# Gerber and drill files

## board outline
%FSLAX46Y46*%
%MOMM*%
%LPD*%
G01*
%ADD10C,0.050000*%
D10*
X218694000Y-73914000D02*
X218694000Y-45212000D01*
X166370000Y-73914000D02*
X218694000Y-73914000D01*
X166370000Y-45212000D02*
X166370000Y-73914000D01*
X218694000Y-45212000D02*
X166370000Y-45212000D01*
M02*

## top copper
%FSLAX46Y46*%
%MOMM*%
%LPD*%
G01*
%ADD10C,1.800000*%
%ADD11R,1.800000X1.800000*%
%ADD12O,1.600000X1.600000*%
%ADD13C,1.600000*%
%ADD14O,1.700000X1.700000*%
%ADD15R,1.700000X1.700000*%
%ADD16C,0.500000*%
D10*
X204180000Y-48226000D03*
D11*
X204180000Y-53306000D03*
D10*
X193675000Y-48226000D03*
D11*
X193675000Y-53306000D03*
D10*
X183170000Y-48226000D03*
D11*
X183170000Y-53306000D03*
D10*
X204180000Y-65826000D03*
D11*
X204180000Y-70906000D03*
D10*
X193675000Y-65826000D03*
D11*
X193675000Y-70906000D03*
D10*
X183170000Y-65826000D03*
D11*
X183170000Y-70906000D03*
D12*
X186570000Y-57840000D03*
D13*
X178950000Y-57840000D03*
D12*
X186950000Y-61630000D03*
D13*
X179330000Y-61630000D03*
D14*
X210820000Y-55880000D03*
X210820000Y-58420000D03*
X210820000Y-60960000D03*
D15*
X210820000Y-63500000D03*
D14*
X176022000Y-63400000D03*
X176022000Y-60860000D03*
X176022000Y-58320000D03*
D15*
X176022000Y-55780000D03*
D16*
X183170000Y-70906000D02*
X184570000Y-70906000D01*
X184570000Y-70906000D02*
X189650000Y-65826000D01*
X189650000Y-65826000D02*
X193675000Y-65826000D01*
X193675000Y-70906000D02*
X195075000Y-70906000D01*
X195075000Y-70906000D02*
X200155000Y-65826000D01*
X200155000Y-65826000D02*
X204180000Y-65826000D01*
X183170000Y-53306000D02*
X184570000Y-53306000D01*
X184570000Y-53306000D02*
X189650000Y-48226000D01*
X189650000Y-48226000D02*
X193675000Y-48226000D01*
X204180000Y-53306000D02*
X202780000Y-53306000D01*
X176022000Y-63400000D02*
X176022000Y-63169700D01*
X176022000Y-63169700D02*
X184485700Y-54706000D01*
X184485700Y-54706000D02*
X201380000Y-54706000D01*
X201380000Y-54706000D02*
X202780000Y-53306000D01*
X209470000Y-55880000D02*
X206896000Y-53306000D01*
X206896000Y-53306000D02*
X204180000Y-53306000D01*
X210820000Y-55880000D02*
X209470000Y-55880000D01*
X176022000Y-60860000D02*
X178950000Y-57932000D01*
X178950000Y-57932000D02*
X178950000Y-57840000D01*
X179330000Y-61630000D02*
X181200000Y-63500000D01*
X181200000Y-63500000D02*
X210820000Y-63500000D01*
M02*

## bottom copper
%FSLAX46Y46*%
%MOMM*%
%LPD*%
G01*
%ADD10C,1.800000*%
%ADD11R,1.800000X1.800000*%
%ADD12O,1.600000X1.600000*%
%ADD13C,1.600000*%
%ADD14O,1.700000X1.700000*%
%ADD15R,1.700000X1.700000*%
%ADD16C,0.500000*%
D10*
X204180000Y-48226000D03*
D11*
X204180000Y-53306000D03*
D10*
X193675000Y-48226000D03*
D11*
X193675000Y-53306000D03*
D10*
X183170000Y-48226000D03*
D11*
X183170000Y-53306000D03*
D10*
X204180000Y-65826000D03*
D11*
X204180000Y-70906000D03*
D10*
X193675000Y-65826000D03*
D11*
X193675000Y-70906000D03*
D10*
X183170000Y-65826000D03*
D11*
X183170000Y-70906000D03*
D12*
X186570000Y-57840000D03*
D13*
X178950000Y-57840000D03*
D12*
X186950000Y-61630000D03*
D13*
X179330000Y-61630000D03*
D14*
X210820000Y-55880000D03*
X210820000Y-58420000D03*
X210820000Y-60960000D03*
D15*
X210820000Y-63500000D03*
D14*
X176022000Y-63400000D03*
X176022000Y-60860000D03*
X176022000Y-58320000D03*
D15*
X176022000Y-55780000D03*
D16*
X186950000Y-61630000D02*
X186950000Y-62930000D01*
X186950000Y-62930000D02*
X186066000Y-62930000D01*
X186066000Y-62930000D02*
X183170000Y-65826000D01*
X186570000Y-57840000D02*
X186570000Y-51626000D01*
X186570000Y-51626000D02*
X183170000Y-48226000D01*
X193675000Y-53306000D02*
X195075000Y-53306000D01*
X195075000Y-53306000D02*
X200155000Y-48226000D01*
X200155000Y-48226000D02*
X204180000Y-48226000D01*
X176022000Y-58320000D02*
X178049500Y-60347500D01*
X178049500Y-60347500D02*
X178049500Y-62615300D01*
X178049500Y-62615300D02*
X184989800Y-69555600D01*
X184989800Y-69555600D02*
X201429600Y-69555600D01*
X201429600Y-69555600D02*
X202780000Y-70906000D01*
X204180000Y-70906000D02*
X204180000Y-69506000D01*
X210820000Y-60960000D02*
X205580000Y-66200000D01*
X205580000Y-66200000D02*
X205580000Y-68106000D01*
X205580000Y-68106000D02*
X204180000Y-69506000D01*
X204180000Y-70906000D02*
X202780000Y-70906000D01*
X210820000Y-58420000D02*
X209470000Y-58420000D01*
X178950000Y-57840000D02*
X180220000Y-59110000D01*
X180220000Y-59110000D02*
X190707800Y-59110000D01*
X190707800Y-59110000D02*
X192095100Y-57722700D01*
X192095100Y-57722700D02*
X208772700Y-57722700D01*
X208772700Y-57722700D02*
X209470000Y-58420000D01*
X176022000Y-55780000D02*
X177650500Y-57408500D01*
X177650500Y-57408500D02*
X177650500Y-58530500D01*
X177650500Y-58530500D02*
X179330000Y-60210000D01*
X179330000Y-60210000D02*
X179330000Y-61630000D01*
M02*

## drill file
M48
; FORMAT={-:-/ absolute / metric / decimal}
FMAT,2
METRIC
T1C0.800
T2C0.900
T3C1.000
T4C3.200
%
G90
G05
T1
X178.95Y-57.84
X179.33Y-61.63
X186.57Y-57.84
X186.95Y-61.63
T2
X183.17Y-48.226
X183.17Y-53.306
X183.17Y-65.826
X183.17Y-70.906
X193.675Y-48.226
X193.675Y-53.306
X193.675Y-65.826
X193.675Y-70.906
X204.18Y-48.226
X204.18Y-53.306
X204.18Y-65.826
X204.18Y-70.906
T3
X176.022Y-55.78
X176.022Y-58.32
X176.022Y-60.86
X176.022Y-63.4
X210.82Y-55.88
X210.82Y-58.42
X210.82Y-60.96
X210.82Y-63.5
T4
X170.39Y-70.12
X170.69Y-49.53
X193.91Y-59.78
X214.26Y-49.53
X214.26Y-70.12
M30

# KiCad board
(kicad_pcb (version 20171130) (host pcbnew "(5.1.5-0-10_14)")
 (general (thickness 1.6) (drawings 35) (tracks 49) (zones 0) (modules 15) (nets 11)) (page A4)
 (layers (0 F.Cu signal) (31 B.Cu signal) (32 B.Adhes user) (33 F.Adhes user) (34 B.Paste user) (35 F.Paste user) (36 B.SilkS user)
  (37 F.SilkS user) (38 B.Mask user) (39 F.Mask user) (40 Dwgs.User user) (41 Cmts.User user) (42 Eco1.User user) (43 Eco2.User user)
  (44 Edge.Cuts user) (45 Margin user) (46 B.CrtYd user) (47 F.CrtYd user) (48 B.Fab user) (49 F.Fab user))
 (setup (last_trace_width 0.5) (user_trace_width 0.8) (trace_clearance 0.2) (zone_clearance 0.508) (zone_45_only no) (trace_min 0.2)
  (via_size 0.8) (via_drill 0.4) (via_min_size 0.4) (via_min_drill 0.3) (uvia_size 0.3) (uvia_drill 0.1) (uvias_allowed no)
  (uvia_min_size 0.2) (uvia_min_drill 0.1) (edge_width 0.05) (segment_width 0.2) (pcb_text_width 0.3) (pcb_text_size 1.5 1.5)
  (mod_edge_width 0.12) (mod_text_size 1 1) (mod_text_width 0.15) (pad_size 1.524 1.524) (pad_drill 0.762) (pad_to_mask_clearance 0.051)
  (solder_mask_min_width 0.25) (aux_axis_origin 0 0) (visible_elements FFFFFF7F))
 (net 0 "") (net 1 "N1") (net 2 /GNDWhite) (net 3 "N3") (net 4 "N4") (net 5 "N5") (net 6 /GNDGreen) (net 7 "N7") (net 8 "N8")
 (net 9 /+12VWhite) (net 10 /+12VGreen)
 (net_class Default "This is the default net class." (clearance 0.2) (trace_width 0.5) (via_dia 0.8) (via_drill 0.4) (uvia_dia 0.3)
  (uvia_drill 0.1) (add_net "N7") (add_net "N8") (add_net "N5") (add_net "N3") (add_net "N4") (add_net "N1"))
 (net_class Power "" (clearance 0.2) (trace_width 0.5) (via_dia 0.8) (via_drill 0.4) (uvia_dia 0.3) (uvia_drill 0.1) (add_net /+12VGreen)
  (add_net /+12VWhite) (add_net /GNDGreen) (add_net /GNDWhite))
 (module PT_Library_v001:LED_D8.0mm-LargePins (layer F.Cu) (at 204.18 53.306 90)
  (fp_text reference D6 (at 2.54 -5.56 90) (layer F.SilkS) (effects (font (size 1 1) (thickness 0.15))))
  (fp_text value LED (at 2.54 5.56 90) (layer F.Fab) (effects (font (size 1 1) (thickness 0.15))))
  (pad 2 thru_hole circle (at 5.08 0 90) (size 1.8 1.8) (drill 0.9) (layers *.Cu *.Mask) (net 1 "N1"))
  (pad 1 thru_hole rect (at 0 0 90) (size 1.8 1.8) (drill 0.9) (layers *.Cu *.Mask) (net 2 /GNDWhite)))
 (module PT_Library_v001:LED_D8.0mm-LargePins (layer F.Cu) (at 193.675 53.306 90)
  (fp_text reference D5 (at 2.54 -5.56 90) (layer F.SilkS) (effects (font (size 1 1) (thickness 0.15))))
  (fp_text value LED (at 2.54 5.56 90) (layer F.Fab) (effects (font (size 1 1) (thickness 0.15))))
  (pad 2 thru_hole circle (at 5.08 0 90) (size 1.8 1.8) (drill 0.9) (layers *.Cu *.Mask) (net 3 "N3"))
  (pad 1 thru_hole rect (at 0 0 90) (size 1.8 1.8) (drill 0.9) (layers *.Cu *.Mask) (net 1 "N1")))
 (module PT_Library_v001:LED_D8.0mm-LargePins (layer F.Cu) (at 183.17 53.306 90)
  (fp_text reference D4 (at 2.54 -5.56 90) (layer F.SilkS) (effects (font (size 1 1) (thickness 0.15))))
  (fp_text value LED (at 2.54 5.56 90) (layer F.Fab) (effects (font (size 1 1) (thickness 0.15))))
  (pad 2 thru_hole circle (at 5.08 0 90) (size 1.8 1.8) (drill 0.9) (layers *.Cu *.Mask) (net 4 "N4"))
  (pad 1 thru_hole rect (at 0 0 90) (size 1.8 1.8) (drill 0.9) (layers *.Cu *.Mask) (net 3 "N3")))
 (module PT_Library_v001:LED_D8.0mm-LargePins (layer F.Cu) (at 204.18 70.906 90)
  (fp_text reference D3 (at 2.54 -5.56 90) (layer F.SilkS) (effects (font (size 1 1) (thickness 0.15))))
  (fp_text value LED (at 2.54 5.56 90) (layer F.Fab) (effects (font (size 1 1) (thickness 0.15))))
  (pad 2 thru_hole circle (at 5.08 0 90) (size 1.8 1.8) (drill 0.9) (layers *.Cu *.Mask) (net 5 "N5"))
  (pad 1 thru_hole rect (at 0 0 90) (size 1.8 1.8) (drill 0.9) (layers *.Cu *.Mask) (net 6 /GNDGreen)))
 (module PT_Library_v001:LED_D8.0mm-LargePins (layer F.Cu) (at 193.675 70.906 90)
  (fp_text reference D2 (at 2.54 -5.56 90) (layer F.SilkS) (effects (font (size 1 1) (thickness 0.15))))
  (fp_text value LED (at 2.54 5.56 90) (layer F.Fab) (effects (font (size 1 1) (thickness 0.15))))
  (pad 2 thru_hole circle (at 5.08 0 90) (size 1.8 1.8) (drill 0.9) (layers *.Cu *.Mask) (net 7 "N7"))
  (pad 1 thru_hole rect (at 0 0 90) (size 1.8 1.8) (drill 0.9) (layers *.Cu *.Mask) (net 5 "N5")))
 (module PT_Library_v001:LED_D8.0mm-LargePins (layer F.Cu) (at 183.17 70.906 90)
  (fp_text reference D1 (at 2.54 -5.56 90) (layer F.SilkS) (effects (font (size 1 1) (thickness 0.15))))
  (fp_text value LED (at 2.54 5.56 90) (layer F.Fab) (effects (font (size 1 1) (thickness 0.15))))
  (pad 2 thru_hole circle (at 5.08 0 90) (size 1.8 1.8) (drill 0.9) (layers *.Cu *.Mask) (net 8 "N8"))
  (pad 1 thru_hole rect (at 0 0 90) (size 1.8 1.8) (drill 0.9) (layers *.Cu *.Mask) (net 7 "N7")))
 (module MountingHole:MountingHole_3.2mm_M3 (layer F.Cu) (at 193.91 59.78)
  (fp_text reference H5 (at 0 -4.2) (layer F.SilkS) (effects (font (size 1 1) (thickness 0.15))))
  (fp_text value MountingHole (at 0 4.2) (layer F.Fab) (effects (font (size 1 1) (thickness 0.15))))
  (pad 1 np_thru_hole circle (at 0 0) (size 3.2 3.2) (drill 3.2) (layers *.Cu *.Mask)))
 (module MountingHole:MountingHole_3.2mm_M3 (layer F.Cu) (at 214.26 70.12)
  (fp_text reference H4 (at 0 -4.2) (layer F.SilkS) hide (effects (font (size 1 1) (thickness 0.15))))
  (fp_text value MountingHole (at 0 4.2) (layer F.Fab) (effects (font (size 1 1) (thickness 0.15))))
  (pad 1 np_thru_hole circle (at 0 0) (size 3.2 3.2) (drill 3.2) (layers *.Cu *.Mask)))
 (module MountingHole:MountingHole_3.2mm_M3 (layer F.Cu) (at 170.39 70.12)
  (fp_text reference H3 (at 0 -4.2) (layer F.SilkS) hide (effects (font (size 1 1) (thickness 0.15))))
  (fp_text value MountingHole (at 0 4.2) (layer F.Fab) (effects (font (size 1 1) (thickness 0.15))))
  (pad 1 np_thru_hole circle (at 0 0) (size 3.2 3.2) (drill 3.2) (layers *.Cu *.Mask)))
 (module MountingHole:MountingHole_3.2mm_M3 (layer F.Cu) (at 214.26 49.53)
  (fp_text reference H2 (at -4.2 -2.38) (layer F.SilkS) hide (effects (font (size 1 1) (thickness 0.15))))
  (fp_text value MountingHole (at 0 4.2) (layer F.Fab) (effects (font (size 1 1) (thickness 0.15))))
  (pad 1 np_thru_hole circle (at 0 0) (size 3.2 3.2) (drill 3.2) (layers *.Cu *.Mask)))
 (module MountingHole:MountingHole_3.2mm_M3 (layer F.Cu) (at 170.69 49.53)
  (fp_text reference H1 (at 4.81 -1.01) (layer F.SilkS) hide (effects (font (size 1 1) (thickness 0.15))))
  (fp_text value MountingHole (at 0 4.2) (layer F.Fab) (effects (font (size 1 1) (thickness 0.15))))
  (pad 1 np_thru_hole circle (at 0 0) (size 3.2 3.2) (drill 3.2) (layers *.Cu *.Mask)))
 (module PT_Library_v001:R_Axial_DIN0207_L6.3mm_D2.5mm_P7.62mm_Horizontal (layer B.Cu) (at 178.95 57.84)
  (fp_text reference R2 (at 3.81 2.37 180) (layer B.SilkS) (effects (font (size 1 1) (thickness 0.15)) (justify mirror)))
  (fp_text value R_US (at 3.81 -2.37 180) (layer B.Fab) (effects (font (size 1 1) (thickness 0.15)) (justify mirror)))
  (pad 2 thru_hole oval (at 7.62 0) (size 1.6 1.6) (drill 0.8) (layers *.Cu *.Mask) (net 4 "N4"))
  (pad 1 thru_hole circle (at 0 0) (size 1.6 1.6) (drill 0.8) (layers *.Cu *.Mask) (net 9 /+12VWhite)))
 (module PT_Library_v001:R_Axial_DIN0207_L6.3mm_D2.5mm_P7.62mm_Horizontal (layer B.Cu) (at 179.33 61.63)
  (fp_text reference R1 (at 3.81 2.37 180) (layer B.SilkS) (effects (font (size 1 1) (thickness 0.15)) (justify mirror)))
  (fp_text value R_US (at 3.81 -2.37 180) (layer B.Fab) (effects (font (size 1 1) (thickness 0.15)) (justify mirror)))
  (pad 2 thru_hole oval (at 7.62 0) (size 1.6 1.6) (drill 0.8) (layers *.Cu *.Mask) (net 8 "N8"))
  (pad 1 thru_hole circle (at 0 0) (size 1.6 1.6) (drill 0.8) (layers *.Cu *.Mask) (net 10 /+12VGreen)))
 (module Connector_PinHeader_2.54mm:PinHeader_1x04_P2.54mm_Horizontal (layer B.Cu) (at 210.82 63.5)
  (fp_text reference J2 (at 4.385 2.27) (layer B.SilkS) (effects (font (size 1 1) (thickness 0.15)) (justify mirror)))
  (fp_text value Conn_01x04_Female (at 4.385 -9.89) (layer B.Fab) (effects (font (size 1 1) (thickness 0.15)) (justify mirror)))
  (pad 4 thru_hole oval (at 0 -7.62) (size 1.7 1.7) (drill 1) (layers *.Cu *.Mask) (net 2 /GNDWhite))
  (pad 3 thru_hole oval (at 0 -5.08) (size 1.7 1.7) (drill 1) (layers *.Cu *.Mask) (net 9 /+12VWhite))
  (pad 2 thru_hole oval (at 0 -2.54) (size 1.7 1.7) (drill 1) (layers *.Cu *.Mask) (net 6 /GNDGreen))
  (pad 1 thru_hole rect (at 0 0) (size 1.7 1.7) (drill 1) (layers *.Cu *.Mask) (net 10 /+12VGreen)))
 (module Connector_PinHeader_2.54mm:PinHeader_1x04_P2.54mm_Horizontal (layer B.Cu) (at 176.022 55.78 180)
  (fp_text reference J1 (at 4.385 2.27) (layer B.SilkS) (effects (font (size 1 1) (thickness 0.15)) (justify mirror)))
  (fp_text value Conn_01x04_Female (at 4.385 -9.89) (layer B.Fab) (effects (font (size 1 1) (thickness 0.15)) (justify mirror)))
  (pad 4 thru_hole oval (at 0 -7.62 180) (size 1.7 1.7) (drill 1) (layers *.Cu *.Mask) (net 2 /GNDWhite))
  (pad 3 thru_hole oval (at 0 -5.08 180) (size 1.7 1.7) (drill 1) (layers *.Cu *.Mask) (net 9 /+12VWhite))
  (pad 2 thru_hole oval (at 0 -2.54 180) (size 1.7 1.7) (drill 1) (layers *.Cu *.Mask) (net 6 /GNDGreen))
  (pad 1 thru_hole rect (at 0 0 180) (size 1.7 1.7) (drill 1) (layers *.Cu *.Mask) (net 10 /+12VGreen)))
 (gr_line (start 218.694 73.914) (end 218.694 45.212) (layer Edge.Cuts) (width 0.05))
 (gr_line (start 166.37 73.914) (end 218.694 73.914) (layer Edge.Cuts) (width 0.05))
 (gr_line (start 166.37 45.212) (end 166.37 73.914) (layer Edge.Cuts) (width 0.05))
 (gr_line (start 218.694 45.212) (end 166.37 45.212) (layer Edge.Cuts) (width 0.05))
 (segment (start 183.17 70.906) (end 184.57 70.906) (width 0.5) (layer F.Cu) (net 7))
 (segment (start 184.57 70.906) (end 189.65 65.826) (width 0.5) (layer F.Cu) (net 7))
 (segment (start 189.65 65.826) (end 193.675 65.826) (width 0.5) (layer F.Cu) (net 7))
 (segment (start 186.95 61.63) (end 186.95 62.93) (width 0.5) (layer B.Cu) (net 8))
 (segment (start 186.95 62.93) (end 186.066 62.93) (width 0.5) (layer B.Cu) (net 8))
 (segment (start 186.066 62.93) (end 183.17 65.826) (width 0.5) (layer B.Cu) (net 8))
 (segment (start 193.675 70.906) (end 195.075 70.906) (width 0.5) (layer F.Cu) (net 5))
 (segment (start 195.075 70.906) (end 200.155 65.826) (width 0.5) (layer F.Cu) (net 5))
 (segment (start 200.155 65.826) (end 204.18 65.826) (width 0.5) (layer F.Cu) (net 5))
 (segment (start 186.57 57.84) (end 186.57 51.626) (width 0.5) (layer B.Cu) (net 4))
 (segment (start 186.57 51.626) (end 183.17 48.226) (width 0.5) (layer B.Cu) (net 4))
 (segment (start 183.17 53.306) (end 184.57 53.306) (width 0.5) (layer F.Cu) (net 3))
 (segment (start 184.57 53.306) (end 189.65 48.226) (width 0.5) (layer F.Cu) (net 3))
 (segment (start 189.65 48.226) (end 193.675 48.226) (width 0.5) (layer F.Cu) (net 3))
 (segment (start 193.675 53.306) (end 195.075 53.306) (width 0.5) (layer B.Cu) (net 1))
 (segment (start 195.075 53.306) (end 200.155 48.226) (width 0.5) (layer B.Cu) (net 1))
 (segment (start 200.155 48.226) (end 204.18 48.226) (width 0.5) (layer B.Cu) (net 1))
 (segment (start 176.022 58.32) (end 178.0495 60.3475) (width 0.5) (layer B.Cu) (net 6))
 (segment (start 178.0495 60.3475) (end 178.0495 62.6153) (width 0.5) (layer B.Cu) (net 6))
 (segment (start 178.0495 62.6153) (end 184.9898 69.5556) (width 0.5) (layer B.Cu) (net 6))
 (segment (start 184.9898 69.5556) (end 201.4296 69.5556) (width 0.5) (layer B.Cu) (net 6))
 (segment (start 201.4296 69.5556) (end 202.78 70.906) (width 0.5) (layer B.Cu) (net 6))
 (segment (start 204.18 70.906) (end 204.18 69.506) (width 0.5) (layer B.Cu) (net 6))
 (segment (start 210.82 60.96) (end 205.58 66.2) (width 0.5) (layer B.Cu) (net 6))
 (segment (start 205.58 66.2) (end 205.58 68.106) (width 0.5) (layer B.Cu) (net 6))
 (segment (start 205.58 68.106) (end 204.18 69.506) (width 0.5) (layer B.Cu) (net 6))
 (segment (start 204.18 70.906) (end 202.78 70.906) (width 0.5) (layer B.Cu) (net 6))
 (segment (start 204.18 53.306) (end 202.78 53.306) (width 0.5) (layer F.Cu) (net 2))
 (segment (start 176.022 63.4) (end 176.022 63.1697) (width 0.5) (layer F.Cu) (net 2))
 (segment (start 176.022 63.1697) (end 184.4857 54.706) (width 0.5) (layer F.Cu) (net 2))
 (segment (start 184.4857 54.706) (end 201.38 54.706) (width 0.5) (layer F.Cu) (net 2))
 (segment (start 201.38 54.706) (end 202.78 53.306) (width 0.5) (layer F.Cu) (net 2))
 (segment (start 209.47 55.88) (end 206.896 53.306) (width 0.5) (layer F.Cu) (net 2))
 (segment (start 206.896 53.306) (end 204.18 53.306) (width 0.5) (layer F.Cu) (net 2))
 (segment (start 210.82 55.88) (end 209.47 55.88) (width 0.5) (layer F.Cu) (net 2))
 (segment (start 210.82 58.42) (end 209.47 58.42) (width 0.5) (layer B.Cu) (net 9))
 (segment (start 178.95 57.84) (end 180.22 59.11) (width 0.5) (layer B.Cu) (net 9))
 (segment (start 180.22 59.11) (end 190.7078 59.11) (width 0.5) (layer B.Cu) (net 9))
 (segment (start 190.7078 59.11) (end 192.0951 57.7227) (width 0.5) (layer B.Cu) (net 9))
 (segment (start 192.0951 57.7227) (end 208.7727 57.7227) (width 0.5) (layer B.Cu) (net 9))
 (segment (start 208.7727 57.7227) (end 209.47 58.42) (width 0.5) (layer B.Cu) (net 9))
 (segment (start 176.022 60.86) (end 178.95 57.932) (width 0.5) (layer F.Cu) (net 9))
 (segment (start 178.95 57.932) (end 178.95 57.84) (width 0.5) (layer F.Cu) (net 9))
 (segment (start 176.022 55.78) (end 177.6505 57.4085) (width 0.5) (layer B.Cu) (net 10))
 (segment (start 177.6505 57.4085) (end 177.6505 58.5305) (width 0.5) (layer B.Cu) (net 10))
 (segment (start 177.6505 58.5305) (end 179.33 60.21) (width 0.5) (layer B.Cu) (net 10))
 (segment (start 179.33 60.21) (end 179.33 61.63) (width 0.5) (layer B.Cu) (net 10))
 (segment (start 179.33 61.63) (end 181.2 63.5) (width 0.5) (layer F.Cu) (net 10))
 (segment (start 181.2 63.5) (end 210.82 63.5) (width 0.5) (layer F.Cu) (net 10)))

